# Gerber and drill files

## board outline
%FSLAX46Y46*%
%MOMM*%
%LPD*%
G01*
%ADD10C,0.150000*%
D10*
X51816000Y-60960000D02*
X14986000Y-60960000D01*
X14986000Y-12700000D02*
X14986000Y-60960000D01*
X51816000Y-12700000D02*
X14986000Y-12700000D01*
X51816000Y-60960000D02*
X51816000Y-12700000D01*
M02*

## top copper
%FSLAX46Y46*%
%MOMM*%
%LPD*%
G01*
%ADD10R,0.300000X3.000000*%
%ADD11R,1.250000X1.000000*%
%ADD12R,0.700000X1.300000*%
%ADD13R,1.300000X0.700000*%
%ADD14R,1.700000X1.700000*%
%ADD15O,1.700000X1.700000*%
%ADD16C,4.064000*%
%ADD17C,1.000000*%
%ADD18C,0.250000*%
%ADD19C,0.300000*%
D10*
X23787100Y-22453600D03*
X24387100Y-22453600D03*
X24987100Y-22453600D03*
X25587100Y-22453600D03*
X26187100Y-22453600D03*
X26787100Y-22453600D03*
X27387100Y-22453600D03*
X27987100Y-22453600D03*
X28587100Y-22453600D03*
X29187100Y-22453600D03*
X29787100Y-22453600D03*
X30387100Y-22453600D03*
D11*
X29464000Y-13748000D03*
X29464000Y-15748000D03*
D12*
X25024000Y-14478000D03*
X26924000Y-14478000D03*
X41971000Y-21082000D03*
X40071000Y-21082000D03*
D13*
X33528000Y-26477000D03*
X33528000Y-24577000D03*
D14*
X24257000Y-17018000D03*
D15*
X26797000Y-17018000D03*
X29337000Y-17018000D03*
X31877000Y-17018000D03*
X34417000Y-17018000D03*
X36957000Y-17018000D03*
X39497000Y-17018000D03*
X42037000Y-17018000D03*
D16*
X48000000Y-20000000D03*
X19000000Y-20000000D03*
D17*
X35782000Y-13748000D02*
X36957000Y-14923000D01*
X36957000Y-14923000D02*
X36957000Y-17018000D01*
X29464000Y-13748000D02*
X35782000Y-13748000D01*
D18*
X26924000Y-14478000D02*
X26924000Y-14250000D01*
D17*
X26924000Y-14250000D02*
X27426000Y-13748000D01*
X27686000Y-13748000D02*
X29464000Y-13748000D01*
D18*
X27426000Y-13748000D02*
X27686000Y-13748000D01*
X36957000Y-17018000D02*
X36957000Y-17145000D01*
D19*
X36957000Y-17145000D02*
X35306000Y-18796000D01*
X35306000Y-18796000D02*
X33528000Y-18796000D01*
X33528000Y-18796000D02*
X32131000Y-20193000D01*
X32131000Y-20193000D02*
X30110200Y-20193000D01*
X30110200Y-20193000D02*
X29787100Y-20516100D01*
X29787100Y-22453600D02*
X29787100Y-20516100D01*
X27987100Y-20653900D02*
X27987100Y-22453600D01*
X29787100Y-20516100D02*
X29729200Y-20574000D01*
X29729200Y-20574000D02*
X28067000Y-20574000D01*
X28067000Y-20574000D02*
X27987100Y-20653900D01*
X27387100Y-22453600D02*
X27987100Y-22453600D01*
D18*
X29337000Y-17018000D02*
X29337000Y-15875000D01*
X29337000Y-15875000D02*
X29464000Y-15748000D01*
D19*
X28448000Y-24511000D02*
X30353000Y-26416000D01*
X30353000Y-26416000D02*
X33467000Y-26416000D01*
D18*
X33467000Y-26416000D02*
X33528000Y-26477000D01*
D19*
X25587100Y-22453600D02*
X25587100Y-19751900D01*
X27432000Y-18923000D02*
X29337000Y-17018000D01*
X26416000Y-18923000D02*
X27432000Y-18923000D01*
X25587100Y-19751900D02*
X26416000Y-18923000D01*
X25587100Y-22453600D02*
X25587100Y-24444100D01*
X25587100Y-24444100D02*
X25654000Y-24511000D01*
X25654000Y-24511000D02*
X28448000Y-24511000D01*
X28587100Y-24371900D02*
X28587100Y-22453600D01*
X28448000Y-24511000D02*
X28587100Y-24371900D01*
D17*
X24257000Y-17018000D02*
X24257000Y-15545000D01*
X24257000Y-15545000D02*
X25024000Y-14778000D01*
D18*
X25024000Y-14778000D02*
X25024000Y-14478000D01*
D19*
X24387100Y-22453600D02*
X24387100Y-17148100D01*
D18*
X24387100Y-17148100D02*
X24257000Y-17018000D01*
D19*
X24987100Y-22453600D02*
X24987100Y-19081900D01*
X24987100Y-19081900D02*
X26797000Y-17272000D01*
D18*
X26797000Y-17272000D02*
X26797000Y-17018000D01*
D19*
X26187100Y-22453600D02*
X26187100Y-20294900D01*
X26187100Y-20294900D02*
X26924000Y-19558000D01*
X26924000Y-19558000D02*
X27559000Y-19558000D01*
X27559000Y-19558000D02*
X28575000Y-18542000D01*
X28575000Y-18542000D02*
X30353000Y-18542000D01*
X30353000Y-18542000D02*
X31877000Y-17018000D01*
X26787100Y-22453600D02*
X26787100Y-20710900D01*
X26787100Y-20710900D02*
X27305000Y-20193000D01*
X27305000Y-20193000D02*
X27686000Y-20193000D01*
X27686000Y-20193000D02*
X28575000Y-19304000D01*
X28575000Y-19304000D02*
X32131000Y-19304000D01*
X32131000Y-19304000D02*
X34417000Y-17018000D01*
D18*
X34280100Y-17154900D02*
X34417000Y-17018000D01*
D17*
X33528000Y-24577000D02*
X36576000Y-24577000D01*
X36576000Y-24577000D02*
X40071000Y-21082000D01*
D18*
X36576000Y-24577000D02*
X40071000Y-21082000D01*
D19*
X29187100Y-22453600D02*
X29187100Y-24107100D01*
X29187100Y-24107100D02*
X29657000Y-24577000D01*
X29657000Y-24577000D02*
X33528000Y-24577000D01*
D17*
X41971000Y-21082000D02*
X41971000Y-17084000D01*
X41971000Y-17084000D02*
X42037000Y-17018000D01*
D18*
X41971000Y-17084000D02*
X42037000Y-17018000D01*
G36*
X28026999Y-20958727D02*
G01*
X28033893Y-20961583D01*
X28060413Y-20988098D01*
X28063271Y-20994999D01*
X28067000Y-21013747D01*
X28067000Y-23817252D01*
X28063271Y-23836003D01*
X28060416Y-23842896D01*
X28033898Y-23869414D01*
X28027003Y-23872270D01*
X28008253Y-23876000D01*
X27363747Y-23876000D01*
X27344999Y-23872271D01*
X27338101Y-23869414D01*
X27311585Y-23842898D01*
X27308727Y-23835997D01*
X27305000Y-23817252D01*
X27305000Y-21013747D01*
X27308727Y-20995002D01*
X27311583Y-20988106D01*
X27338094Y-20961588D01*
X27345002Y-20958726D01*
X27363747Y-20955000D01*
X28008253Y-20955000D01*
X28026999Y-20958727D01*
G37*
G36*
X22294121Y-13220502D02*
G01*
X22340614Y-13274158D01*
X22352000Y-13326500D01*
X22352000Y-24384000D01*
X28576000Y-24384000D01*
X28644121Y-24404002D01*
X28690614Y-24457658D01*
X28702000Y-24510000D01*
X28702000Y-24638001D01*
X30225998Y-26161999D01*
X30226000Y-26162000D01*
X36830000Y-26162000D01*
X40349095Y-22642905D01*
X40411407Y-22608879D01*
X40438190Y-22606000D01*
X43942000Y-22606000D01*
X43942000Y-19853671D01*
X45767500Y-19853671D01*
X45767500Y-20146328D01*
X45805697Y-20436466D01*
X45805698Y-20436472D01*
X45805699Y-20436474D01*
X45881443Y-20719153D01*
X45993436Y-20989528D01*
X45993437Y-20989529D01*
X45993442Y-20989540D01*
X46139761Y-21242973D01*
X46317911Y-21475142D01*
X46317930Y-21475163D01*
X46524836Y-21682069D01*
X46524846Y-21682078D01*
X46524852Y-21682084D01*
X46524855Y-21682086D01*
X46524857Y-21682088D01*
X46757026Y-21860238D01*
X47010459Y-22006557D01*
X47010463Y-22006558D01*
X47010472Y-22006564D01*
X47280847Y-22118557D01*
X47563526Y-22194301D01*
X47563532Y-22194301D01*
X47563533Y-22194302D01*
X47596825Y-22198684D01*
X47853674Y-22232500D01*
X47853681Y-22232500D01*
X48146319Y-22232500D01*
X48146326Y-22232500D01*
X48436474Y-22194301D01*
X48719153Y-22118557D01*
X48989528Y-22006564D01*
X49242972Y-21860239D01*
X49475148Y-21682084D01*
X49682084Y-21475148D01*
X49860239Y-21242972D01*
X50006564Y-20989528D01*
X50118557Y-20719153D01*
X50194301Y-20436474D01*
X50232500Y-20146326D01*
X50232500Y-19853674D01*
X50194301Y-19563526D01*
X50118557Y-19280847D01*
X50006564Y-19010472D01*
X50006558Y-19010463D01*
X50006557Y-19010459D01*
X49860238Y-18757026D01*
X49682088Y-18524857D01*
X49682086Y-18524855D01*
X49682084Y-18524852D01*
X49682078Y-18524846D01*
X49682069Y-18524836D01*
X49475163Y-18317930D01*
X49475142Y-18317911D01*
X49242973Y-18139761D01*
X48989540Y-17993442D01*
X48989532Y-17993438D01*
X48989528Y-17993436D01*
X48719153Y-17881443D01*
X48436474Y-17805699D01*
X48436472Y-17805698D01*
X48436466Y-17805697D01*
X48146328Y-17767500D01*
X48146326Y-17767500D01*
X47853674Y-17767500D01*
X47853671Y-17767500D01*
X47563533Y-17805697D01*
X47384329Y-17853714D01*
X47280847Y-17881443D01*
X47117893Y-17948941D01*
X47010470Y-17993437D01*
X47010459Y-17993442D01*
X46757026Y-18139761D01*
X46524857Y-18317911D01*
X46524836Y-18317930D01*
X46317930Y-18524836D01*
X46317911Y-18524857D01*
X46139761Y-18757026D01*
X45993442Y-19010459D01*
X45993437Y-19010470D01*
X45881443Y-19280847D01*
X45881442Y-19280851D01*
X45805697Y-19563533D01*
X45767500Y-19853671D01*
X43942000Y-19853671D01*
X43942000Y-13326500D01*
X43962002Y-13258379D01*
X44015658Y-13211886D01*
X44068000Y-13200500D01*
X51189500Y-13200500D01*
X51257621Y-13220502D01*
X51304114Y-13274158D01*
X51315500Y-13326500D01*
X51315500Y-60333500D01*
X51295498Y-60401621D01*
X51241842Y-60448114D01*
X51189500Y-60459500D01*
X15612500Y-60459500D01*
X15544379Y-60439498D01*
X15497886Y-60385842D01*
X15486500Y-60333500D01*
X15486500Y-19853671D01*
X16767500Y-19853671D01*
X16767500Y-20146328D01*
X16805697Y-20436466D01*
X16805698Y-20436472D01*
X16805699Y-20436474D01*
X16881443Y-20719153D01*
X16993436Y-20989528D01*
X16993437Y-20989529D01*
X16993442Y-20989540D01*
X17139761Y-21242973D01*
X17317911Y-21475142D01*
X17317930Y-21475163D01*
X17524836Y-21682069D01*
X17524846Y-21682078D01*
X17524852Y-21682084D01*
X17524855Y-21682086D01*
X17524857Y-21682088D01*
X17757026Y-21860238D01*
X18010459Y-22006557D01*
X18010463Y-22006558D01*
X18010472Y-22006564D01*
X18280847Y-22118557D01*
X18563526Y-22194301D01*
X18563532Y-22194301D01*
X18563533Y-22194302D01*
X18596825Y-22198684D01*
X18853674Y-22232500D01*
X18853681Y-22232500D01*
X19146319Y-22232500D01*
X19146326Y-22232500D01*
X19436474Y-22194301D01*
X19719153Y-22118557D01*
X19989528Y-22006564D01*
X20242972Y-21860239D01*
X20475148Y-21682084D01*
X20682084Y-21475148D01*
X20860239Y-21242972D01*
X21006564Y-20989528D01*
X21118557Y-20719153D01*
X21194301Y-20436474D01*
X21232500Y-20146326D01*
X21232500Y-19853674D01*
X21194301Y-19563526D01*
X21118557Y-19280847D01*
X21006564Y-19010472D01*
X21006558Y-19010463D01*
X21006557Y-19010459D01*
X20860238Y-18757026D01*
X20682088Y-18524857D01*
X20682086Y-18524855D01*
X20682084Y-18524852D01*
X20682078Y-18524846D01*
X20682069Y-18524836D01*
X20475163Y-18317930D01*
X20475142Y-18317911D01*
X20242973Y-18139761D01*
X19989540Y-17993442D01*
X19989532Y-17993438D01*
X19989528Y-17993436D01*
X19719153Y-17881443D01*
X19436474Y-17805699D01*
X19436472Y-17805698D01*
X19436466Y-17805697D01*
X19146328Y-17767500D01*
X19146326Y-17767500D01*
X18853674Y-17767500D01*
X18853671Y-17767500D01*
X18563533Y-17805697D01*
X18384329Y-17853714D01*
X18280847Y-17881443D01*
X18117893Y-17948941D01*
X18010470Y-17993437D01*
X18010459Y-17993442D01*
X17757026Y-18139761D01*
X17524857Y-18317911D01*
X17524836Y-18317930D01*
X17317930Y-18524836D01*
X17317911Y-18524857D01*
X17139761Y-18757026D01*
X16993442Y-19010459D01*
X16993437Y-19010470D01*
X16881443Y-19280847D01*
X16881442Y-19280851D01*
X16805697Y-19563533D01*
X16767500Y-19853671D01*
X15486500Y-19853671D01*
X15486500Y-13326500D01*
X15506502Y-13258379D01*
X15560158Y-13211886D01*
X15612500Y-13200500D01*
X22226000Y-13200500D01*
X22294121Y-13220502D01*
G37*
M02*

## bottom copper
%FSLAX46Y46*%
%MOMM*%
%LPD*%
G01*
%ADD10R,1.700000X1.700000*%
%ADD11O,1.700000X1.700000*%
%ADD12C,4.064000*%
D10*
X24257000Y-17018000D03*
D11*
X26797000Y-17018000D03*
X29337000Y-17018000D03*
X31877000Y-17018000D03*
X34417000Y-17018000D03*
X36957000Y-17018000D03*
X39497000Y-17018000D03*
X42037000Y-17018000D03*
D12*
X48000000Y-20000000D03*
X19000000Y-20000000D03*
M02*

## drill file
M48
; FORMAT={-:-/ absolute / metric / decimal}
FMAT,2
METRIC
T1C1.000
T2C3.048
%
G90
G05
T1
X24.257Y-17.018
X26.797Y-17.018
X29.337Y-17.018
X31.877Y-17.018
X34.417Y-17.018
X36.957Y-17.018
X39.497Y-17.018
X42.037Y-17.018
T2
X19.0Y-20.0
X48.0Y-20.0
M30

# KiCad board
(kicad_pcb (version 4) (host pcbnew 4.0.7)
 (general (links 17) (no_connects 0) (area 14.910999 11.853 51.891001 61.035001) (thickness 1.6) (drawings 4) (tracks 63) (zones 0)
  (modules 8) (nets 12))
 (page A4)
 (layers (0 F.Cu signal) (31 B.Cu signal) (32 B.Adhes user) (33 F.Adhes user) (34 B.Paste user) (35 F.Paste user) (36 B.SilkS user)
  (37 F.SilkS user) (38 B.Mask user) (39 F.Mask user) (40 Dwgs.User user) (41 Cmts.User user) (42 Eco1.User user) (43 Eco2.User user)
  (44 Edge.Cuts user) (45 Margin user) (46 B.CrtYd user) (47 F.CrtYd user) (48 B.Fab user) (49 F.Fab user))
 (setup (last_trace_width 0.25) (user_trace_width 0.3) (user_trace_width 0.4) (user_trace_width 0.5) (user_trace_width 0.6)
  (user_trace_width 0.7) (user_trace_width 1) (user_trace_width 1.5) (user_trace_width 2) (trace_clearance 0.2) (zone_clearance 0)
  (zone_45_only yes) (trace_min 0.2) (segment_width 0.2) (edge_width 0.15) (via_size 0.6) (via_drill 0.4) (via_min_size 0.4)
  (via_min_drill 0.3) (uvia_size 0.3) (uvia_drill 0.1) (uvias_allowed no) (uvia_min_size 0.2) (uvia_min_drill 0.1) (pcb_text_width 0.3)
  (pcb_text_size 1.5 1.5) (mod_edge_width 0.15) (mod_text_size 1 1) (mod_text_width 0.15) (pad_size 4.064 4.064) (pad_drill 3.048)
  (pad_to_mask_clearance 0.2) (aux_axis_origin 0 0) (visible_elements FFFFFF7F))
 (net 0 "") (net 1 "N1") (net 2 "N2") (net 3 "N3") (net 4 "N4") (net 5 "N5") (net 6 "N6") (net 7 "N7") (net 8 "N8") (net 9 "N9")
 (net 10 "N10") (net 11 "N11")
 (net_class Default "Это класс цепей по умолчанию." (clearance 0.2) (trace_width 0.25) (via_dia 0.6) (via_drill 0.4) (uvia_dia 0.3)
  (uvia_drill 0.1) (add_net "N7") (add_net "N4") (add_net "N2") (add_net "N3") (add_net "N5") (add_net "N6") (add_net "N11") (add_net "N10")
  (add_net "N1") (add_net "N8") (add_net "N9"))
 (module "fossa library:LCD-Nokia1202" (layer F.Cu) (at 15.4051 23.2156)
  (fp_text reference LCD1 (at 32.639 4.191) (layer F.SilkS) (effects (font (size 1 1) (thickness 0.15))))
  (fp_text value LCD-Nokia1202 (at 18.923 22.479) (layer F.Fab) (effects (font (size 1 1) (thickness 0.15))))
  (pad 1 smd rect (at 8.382 -0.762) (size 0.3 3) (layers F.Cu F.Paste F.Mask) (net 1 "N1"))
  (pad 2 smd rect (at 8.982 -0.762) (size 0.3 3) (layers F.Cu F.Paste F.Mask) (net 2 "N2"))
  (pad 3 smd rect (at 9.582 -0.762) (size 0.3 3) (layers F.Cu F.Paste F.Mask) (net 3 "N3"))
  (pad 4 smd rect (at 10.182 -0.762) (size 0.3 3) (layers F.Cu F.Paste F.Mask) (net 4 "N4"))
  (pad 5 smd rect (at 10.782 -0.762) (size 0.3 3) (layers F.Cu F.Paste F.Mask) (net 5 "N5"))
  (pad 6 smd rect (at 11.382 -0.762) (size 0.3 3) (layers F.Cu F.Paste F.Mask) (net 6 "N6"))
  (pad 7 smd rect (at 11.982 -0.762) (size 0.3 3) (layers F.Cu F.Paste F.Mask) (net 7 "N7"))
  (pad 8 smd rect (at 12.582 -0.762) (size 0.3 3) (layers F.Cu F.Paste F.Mask) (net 7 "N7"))
  (pad 9 smd rect (at 13.182 -0.762) (size 0.3 3) (layers F.Cu F.Paste F.Mask) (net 4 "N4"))
  (pad 10 smd rect (at 13.782 -0.762) (size 0.3 3) (layers F.Cu F.Paste F.Mask) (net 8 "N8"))
  (pad 11 smd rect (at 14.382 -0.762) (size 0.3 3) (layers F.Cu F.Paste F.Mask) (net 7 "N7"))
  (pad 12 smd rect (at 14.982 -0.762) (size 0.3 3) (layers F.Cu F.Paste F.Mask) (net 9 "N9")))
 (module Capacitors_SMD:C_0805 (layer F.Cu) (at 29.464 14.748 270)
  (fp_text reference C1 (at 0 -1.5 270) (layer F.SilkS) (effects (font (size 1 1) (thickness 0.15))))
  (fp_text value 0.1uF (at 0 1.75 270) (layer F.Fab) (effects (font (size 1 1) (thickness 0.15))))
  (pad 1 smd rect (at -1 0 270) (size 1 1.25) (layers F.Cu F.Paste F.Mask) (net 7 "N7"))
  (pad 2 smd rect (at 1 0 270) (size 1 1.25) (layers F.Cu F.Paste F.Mask) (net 4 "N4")))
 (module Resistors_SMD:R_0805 (layer F.Cu) (at 25.974 14.478)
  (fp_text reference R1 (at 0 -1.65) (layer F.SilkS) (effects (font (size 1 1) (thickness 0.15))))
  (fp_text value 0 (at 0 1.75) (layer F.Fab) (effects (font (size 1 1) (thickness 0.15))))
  (pad 1 smd rect (at -0.95 0) (size 0.7 1.3) (layers F.Cu F.Paste F.Mask) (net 2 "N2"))
  (pad 2 smd rect (at 0.95 0) (size 0.7 1.3) (layers F.Cu F.Paste F.Mask) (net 7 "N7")))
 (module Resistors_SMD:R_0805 (layer F.Cu) (at 41.021 21.082 180)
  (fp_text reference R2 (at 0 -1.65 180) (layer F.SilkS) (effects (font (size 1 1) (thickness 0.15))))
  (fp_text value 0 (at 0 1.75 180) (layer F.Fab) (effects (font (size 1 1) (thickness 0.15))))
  (pad 1 smd rect (at -0.95 0 180) (size 0.7 1.3) (layers F.Cu F.Paste F.Mask) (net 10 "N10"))
  (pad 2 smd rect (at 0.95 0 180) (size 0.7 1.3) (layers F.Cu F.Paste F.Mask) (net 8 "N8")))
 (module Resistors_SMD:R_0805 (layer F.Cu) (at 33.528 25.527 90)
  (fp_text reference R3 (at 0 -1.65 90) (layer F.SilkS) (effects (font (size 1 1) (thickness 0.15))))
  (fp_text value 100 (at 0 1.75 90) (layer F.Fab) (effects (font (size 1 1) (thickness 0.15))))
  (pad 1 smd rect (at -0.95 0 90) (size 0.7 1.3) (layers F.Cu F.Paste F.Mask) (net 4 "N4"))
  (pad 2 smd rect (at 0.95 0 90) (size 0.7 1.3) (layers F.Cu F.Paste F.Mask) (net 8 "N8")))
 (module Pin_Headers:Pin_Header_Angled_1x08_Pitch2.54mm (layer B.Cu) (at 24.257 17.018 270)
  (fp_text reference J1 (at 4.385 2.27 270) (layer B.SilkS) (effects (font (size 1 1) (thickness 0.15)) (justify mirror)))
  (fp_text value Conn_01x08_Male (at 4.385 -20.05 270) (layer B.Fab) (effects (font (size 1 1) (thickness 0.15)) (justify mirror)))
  (pad 1 thru_hole rect (at 0 0 270) (size 1.7 1.7) (drill 1) (layers *.Cu *.Mask) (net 2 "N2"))
  (pad 2 thru_hole oval (at 0 -2.54 270) (size 1.7 1.7) (drill 1) (layers *.Cu *.Mask) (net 3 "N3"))
  (pad 3 thru_hole oval (at 0 -5.08 270) (size 1.7 1.7) (drill 1) (layers *.Cu *.Mask) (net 4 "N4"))
  (pad 4 thru_hole oval (at 0 -7.62 270) (size 1.7 1.7) (drill 1) (layers *.Cu *.Mask) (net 5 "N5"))
  (pad 5 thru_hole oval (at 0 -10.16 270) (size 1.7 1.7) (drill 1) (layers *.Cu *.Mask) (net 6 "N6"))
  (pad 6 thru_hole oval (at 0 -12.7 270) (size 1.7 1.7) (drill 1) (layers *.Cu *.Mask) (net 7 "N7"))
  (pad 7 thru_hole oval (at 0 -15.24 270) (size 1.7 1.7) (drill 1) (layers *.Cu *.Mask) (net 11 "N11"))
  (pad 8 thru_hole oval (at 0 -17.78 270) (size 1.7 1.7) (drill 1) (layers *.Cu *.Mask) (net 10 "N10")))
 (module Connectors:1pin (layer F.Cu) (at 48 20)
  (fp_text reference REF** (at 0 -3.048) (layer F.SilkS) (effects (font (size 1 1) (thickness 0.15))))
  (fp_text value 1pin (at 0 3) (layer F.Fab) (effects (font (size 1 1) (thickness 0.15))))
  (pad 1 thru_hole circle (at 0 0) (size 4.064 4.064) (drill 3.048) (layers *.Cu *.Mask)))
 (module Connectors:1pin (layer F.Cu) (at 19 20)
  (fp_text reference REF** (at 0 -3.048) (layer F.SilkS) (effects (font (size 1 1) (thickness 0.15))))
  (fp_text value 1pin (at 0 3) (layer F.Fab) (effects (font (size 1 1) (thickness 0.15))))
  (pad 1 thru_hole circle (at 0 0) (size 4.064 4.064) (drill 3.048) (layers *.Cu *.Mask)))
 (gr_line (start 51.816 60.96) (end 14.986 60.96) (angle 90) (layer Edge.Cuts) (width 0.15))
 (gr_line (start 14.986 12.7) (end 14.986 60.96) (angle 90) (layer Edge.Cuts) (width 0.15))
 (gr_line (start 51.816 12.7) (end 14.986 12.7) (angle 90) (layer Edge.Cuts) (width 0.15))
 (gr_line (start 51.816 60.96) (end 51.816 12.7) (angle 90) (layer Edge.Cuts) (width 0.15))
 (segment (start 35.782 13.748) (end 36.957 14.923) (width 1) (layer F.Cu) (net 7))
 (segment (start 36.957 14.923) (end 36.957 17.018) (width 1) (layer F.Cu) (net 7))
 (segment (start 29.464 13.748) (end 35.782 13.748) (width 1) (layer F.Cu) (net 7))
 (segment (start 26.924 14.478) (end 26.924 14.25) (width 0.25) (layer F.Cu) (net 7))
 (segment (start 26.924 14.25) (end 27.426 13.748) (width 1) (layer F.Cu) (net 7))
 (segment (start 27.686 13.748) (end 29.464 13.748) (width 1) (layer F.Cu) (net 7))
 (segment (start 27.426 13.748) (end 27.686 13.748) (width 0.25) (layer F.Cu) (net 7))
 (segment (start 36.957 17.018) (end 36.957 17.145) (width 0.25) (layer F.Cu) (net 7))
 (segment (start 36.957 17.145) (end 35.306 18.796) (width 0.3) (layer F.Cu) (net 7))
 (segment (start 35.306 18.796) (end 33.528 18.796) (width 0.3) (layer F.Cu) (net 7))
 (segment (start 33.528 18.796) (end 32.131 20.193) (width 0.3) (layer F.Cu) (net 7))
 (segment (start 32.131 20.193) (end 30.1102 20.193) (width 0.3) (layer F.Cu) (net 7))
 (segment (start 30.1102 20.193) (end 29.7871 20.5161) (width 0.3) (layer F.Cu) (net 7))
 (segment (start 29.7871 22.4536) (end 29.7871 20.5161) (width 0.3) (layer F.Cu) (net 7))
 (segment (start 27.9871 20.6539) (end 27.9871 22.4536) (width 0.3) (layer F.Cu) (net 7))
 (segment (start 29.7871 20.5161) (end 29.7292 20.574) (width 0.3) (layer F.Cu) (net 7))
 (segment (start 29.7292 20.574) (end 28.067 20.574) (width 0.3) (layer F.Cu) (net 7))
 (segment (start 28.067 20.574) (end 27.9871 20.6539) (width 0.3) (layer F.Cu) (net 7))
 (segment (start 27.3871 22.4536) (end 27.9871 22.4536) (width 0.3) (layer F.Cu) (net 7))
 (segment (start 29.337 17.018) (end 29.337 15.875) (width 0.25) (layer F.Cu) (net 4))
 (segment (start 29.337 15.875) (end 29.464 15.748) (width 0.25) (layer F.Cu) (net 4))
 (segment (start 28.448 24.511) (end 30.353 26.416) (width 0.3) (layer F.Cu) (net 4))
 (segment (start 30.353 26.416) (end 33.467 26.416) (width 0.3) (layer F.Cu) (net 4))
 (segment (start 33.467 26.416) (end 33.528 26.477) (width 0.25) (layer F.Cu) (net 4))
 (segment (start 25.5871 22.4536) (end 25.5871 19.7519) (width 0.3) (layer F.Cu) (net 4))
 (segment (start 27.432 18.923) (end 29.337 17.018) (width 0.3) (layer F.Cu) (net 4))
 (segment (start 26.416 18.923) (end 27.432 18.923) (width 0.3) (layer F.Cu) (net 4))
 (segment (start 25.5871 19.7519) (end 26.416 18.923) (width 0.3) (layer F.Cu) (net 4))
 (segment (start 25.5871 22.4536) (end 25.5871 24.4441) (width 0.3) (layer F.Cu) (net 4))
 (segment (start 25.5871 24.4441) (end 25.654 24.511) (width 0.3) (layer F.Cu) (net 4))
 (segment (start 25.654 24.511) (end 28.448 24.511) (width 0.3) (layer F.Cu) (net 4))
 (segment (start 28.5871 24.3719) (end 28.5871 22.4536) (width 0.3) (layer F.Cu) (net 4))
 (segment (start 28.448 24.511) (end 28.5871 24.3719) (width 0.3) (layer F.Cu) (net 4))
 (segment (start 24.257 17.018) (end 24.257 15.545) (width 1) (layer F.Cu) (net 2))
 (segment (start 24.257 15.545) (end 25.024 14.778) (width 1) (layer F.Cu) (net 2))
 (segment (start 25.024 14.778) (end 25.024 14.478) (width 0.25) (layer F.Cu) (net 2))
 (segment (start 24.3871 22.4536) (end 24.3871 17.1481) (width 0.3) (layer F.Cu) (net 2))
 (segment (start 24.3871 17.1481) (end 24.257 17.018) (width 0.25) (layer F.Cu) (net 2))
 (segment (start 24.9871 22.4536) (end 24.9871 19.0819) (width 0.3) (layer F.Cu) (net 3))
 (segment (start 24.9871 19.0819) (end 26.797 17.272) (width 0.3) (layer F.Cu) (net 3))
 (segment (start 26.797 17.272) (end 26.797 17.018) (width 0.25) (layer F.Cu) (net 3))
 (segment (start 26.1871 22.4536) (end 26.1871 20.2949) (width 0.3) (layer F.Cu) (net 5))
 (segment (start 26.1871 20.2949) (end 26.924 19.558) (width 0.3) (layer F.Cu) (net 5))
 (segment (start 26.924 19.558) (end 27.559 19.558) (width 0.3) (layer F.Cu) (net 5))
 (segment (start 27.559 19.558) (end 28.575 18.542) (width 0.3) (layer F.Cu) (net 5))
 (segment (start 28.575 18.542) (end 30.353 18.542) (width 0.3) (layer F.Cu) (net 5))
 (segment (start 30.353 18.542) (end 31.877 17.018) (width 0.3) (layer F.Cu) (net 5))
 (segment (start 26.7871 22.4536) (end 26.7871 20.7109) (width 0.3) (layer F.Cu) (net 6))
 (segment (start 26.7871 20.7109) (end 27.305 20.193) (width 0.3) (layer F.Cu) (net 6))
 (segment (start 27.305 20.193) (end 27.686 20.193) (width 0.3) (layer F.Cu) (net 6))
 (segment (start 27.686 20.193) (end 28.575 19.304) (width 0.3) (layer F.Cu) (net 6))
 (segment (start 28.575 19.304) (end 32.131 19.304) (width 0.3) (layer F.Cu) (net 6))
 (segment (start 32.131 19.304) (end 34.417 17.018) (width 0.3) (layer F.Cu) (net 6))
 (segment (start 34.2801 17.1549) (end 34.417 17.018) (width 0.25) (layer F.Cu) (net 6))
 (segment (start 33.528 24.577) (end 36.576 24.577) (width 1) (layer F.Cu) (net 8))
 (segment (start 36.576 24.577) (end 40.071 21.082) (width 1) (layer F.Cu) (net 8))
 (segment (start 36.576 24.577) (end 40.071 21.082) (width 0.25) (layer F.Cu) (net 8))
 (segment (start 29.1871 22.4536) (end 29.1871 24.1071) (width 0.3) (layer F.Cu) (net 8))
 (segment (start 29.1871 24.1071) (end 29.657 24.577) (width 0.3) (layer F.Cu) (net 8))
 (segment (start 29.657 24.577) (end 33.528 24.577) (width 0.3) (layer F.Cu) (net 8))
 (segment (start 41.971 21.082) (end 41.971 17.084) (width 1) (layer F.Cu) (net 10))
 (segment (start 41.971 17.084) (end 42.037 17.018) (width 1) (layer F.Cu) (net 10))
 (segment (start 41.971 17.084) (end 42.037 17.018) (width 0.25) (layer F.Cu) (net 10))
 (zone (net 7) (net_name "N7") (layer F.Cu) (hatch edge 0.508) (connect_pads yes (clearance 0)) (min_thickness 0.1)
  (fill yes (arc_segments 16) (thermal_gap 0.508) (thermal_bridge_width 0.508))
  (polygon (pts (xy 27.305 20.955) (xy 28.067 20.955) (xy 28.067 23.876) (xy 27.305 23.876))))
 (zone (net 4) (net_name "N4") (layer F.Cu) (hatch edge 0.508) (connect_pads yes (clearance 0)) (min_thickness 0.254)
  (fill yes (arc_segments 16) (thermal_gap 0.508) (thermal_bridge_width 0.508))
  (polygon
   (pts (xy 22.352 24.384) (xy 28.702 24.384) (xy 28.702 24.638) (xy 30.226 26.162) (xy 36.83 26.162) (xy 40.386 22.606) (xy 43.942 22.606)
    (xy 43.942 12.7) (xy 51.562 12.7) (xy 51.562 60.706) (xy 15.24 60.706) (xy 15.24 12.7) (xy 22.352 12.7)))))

